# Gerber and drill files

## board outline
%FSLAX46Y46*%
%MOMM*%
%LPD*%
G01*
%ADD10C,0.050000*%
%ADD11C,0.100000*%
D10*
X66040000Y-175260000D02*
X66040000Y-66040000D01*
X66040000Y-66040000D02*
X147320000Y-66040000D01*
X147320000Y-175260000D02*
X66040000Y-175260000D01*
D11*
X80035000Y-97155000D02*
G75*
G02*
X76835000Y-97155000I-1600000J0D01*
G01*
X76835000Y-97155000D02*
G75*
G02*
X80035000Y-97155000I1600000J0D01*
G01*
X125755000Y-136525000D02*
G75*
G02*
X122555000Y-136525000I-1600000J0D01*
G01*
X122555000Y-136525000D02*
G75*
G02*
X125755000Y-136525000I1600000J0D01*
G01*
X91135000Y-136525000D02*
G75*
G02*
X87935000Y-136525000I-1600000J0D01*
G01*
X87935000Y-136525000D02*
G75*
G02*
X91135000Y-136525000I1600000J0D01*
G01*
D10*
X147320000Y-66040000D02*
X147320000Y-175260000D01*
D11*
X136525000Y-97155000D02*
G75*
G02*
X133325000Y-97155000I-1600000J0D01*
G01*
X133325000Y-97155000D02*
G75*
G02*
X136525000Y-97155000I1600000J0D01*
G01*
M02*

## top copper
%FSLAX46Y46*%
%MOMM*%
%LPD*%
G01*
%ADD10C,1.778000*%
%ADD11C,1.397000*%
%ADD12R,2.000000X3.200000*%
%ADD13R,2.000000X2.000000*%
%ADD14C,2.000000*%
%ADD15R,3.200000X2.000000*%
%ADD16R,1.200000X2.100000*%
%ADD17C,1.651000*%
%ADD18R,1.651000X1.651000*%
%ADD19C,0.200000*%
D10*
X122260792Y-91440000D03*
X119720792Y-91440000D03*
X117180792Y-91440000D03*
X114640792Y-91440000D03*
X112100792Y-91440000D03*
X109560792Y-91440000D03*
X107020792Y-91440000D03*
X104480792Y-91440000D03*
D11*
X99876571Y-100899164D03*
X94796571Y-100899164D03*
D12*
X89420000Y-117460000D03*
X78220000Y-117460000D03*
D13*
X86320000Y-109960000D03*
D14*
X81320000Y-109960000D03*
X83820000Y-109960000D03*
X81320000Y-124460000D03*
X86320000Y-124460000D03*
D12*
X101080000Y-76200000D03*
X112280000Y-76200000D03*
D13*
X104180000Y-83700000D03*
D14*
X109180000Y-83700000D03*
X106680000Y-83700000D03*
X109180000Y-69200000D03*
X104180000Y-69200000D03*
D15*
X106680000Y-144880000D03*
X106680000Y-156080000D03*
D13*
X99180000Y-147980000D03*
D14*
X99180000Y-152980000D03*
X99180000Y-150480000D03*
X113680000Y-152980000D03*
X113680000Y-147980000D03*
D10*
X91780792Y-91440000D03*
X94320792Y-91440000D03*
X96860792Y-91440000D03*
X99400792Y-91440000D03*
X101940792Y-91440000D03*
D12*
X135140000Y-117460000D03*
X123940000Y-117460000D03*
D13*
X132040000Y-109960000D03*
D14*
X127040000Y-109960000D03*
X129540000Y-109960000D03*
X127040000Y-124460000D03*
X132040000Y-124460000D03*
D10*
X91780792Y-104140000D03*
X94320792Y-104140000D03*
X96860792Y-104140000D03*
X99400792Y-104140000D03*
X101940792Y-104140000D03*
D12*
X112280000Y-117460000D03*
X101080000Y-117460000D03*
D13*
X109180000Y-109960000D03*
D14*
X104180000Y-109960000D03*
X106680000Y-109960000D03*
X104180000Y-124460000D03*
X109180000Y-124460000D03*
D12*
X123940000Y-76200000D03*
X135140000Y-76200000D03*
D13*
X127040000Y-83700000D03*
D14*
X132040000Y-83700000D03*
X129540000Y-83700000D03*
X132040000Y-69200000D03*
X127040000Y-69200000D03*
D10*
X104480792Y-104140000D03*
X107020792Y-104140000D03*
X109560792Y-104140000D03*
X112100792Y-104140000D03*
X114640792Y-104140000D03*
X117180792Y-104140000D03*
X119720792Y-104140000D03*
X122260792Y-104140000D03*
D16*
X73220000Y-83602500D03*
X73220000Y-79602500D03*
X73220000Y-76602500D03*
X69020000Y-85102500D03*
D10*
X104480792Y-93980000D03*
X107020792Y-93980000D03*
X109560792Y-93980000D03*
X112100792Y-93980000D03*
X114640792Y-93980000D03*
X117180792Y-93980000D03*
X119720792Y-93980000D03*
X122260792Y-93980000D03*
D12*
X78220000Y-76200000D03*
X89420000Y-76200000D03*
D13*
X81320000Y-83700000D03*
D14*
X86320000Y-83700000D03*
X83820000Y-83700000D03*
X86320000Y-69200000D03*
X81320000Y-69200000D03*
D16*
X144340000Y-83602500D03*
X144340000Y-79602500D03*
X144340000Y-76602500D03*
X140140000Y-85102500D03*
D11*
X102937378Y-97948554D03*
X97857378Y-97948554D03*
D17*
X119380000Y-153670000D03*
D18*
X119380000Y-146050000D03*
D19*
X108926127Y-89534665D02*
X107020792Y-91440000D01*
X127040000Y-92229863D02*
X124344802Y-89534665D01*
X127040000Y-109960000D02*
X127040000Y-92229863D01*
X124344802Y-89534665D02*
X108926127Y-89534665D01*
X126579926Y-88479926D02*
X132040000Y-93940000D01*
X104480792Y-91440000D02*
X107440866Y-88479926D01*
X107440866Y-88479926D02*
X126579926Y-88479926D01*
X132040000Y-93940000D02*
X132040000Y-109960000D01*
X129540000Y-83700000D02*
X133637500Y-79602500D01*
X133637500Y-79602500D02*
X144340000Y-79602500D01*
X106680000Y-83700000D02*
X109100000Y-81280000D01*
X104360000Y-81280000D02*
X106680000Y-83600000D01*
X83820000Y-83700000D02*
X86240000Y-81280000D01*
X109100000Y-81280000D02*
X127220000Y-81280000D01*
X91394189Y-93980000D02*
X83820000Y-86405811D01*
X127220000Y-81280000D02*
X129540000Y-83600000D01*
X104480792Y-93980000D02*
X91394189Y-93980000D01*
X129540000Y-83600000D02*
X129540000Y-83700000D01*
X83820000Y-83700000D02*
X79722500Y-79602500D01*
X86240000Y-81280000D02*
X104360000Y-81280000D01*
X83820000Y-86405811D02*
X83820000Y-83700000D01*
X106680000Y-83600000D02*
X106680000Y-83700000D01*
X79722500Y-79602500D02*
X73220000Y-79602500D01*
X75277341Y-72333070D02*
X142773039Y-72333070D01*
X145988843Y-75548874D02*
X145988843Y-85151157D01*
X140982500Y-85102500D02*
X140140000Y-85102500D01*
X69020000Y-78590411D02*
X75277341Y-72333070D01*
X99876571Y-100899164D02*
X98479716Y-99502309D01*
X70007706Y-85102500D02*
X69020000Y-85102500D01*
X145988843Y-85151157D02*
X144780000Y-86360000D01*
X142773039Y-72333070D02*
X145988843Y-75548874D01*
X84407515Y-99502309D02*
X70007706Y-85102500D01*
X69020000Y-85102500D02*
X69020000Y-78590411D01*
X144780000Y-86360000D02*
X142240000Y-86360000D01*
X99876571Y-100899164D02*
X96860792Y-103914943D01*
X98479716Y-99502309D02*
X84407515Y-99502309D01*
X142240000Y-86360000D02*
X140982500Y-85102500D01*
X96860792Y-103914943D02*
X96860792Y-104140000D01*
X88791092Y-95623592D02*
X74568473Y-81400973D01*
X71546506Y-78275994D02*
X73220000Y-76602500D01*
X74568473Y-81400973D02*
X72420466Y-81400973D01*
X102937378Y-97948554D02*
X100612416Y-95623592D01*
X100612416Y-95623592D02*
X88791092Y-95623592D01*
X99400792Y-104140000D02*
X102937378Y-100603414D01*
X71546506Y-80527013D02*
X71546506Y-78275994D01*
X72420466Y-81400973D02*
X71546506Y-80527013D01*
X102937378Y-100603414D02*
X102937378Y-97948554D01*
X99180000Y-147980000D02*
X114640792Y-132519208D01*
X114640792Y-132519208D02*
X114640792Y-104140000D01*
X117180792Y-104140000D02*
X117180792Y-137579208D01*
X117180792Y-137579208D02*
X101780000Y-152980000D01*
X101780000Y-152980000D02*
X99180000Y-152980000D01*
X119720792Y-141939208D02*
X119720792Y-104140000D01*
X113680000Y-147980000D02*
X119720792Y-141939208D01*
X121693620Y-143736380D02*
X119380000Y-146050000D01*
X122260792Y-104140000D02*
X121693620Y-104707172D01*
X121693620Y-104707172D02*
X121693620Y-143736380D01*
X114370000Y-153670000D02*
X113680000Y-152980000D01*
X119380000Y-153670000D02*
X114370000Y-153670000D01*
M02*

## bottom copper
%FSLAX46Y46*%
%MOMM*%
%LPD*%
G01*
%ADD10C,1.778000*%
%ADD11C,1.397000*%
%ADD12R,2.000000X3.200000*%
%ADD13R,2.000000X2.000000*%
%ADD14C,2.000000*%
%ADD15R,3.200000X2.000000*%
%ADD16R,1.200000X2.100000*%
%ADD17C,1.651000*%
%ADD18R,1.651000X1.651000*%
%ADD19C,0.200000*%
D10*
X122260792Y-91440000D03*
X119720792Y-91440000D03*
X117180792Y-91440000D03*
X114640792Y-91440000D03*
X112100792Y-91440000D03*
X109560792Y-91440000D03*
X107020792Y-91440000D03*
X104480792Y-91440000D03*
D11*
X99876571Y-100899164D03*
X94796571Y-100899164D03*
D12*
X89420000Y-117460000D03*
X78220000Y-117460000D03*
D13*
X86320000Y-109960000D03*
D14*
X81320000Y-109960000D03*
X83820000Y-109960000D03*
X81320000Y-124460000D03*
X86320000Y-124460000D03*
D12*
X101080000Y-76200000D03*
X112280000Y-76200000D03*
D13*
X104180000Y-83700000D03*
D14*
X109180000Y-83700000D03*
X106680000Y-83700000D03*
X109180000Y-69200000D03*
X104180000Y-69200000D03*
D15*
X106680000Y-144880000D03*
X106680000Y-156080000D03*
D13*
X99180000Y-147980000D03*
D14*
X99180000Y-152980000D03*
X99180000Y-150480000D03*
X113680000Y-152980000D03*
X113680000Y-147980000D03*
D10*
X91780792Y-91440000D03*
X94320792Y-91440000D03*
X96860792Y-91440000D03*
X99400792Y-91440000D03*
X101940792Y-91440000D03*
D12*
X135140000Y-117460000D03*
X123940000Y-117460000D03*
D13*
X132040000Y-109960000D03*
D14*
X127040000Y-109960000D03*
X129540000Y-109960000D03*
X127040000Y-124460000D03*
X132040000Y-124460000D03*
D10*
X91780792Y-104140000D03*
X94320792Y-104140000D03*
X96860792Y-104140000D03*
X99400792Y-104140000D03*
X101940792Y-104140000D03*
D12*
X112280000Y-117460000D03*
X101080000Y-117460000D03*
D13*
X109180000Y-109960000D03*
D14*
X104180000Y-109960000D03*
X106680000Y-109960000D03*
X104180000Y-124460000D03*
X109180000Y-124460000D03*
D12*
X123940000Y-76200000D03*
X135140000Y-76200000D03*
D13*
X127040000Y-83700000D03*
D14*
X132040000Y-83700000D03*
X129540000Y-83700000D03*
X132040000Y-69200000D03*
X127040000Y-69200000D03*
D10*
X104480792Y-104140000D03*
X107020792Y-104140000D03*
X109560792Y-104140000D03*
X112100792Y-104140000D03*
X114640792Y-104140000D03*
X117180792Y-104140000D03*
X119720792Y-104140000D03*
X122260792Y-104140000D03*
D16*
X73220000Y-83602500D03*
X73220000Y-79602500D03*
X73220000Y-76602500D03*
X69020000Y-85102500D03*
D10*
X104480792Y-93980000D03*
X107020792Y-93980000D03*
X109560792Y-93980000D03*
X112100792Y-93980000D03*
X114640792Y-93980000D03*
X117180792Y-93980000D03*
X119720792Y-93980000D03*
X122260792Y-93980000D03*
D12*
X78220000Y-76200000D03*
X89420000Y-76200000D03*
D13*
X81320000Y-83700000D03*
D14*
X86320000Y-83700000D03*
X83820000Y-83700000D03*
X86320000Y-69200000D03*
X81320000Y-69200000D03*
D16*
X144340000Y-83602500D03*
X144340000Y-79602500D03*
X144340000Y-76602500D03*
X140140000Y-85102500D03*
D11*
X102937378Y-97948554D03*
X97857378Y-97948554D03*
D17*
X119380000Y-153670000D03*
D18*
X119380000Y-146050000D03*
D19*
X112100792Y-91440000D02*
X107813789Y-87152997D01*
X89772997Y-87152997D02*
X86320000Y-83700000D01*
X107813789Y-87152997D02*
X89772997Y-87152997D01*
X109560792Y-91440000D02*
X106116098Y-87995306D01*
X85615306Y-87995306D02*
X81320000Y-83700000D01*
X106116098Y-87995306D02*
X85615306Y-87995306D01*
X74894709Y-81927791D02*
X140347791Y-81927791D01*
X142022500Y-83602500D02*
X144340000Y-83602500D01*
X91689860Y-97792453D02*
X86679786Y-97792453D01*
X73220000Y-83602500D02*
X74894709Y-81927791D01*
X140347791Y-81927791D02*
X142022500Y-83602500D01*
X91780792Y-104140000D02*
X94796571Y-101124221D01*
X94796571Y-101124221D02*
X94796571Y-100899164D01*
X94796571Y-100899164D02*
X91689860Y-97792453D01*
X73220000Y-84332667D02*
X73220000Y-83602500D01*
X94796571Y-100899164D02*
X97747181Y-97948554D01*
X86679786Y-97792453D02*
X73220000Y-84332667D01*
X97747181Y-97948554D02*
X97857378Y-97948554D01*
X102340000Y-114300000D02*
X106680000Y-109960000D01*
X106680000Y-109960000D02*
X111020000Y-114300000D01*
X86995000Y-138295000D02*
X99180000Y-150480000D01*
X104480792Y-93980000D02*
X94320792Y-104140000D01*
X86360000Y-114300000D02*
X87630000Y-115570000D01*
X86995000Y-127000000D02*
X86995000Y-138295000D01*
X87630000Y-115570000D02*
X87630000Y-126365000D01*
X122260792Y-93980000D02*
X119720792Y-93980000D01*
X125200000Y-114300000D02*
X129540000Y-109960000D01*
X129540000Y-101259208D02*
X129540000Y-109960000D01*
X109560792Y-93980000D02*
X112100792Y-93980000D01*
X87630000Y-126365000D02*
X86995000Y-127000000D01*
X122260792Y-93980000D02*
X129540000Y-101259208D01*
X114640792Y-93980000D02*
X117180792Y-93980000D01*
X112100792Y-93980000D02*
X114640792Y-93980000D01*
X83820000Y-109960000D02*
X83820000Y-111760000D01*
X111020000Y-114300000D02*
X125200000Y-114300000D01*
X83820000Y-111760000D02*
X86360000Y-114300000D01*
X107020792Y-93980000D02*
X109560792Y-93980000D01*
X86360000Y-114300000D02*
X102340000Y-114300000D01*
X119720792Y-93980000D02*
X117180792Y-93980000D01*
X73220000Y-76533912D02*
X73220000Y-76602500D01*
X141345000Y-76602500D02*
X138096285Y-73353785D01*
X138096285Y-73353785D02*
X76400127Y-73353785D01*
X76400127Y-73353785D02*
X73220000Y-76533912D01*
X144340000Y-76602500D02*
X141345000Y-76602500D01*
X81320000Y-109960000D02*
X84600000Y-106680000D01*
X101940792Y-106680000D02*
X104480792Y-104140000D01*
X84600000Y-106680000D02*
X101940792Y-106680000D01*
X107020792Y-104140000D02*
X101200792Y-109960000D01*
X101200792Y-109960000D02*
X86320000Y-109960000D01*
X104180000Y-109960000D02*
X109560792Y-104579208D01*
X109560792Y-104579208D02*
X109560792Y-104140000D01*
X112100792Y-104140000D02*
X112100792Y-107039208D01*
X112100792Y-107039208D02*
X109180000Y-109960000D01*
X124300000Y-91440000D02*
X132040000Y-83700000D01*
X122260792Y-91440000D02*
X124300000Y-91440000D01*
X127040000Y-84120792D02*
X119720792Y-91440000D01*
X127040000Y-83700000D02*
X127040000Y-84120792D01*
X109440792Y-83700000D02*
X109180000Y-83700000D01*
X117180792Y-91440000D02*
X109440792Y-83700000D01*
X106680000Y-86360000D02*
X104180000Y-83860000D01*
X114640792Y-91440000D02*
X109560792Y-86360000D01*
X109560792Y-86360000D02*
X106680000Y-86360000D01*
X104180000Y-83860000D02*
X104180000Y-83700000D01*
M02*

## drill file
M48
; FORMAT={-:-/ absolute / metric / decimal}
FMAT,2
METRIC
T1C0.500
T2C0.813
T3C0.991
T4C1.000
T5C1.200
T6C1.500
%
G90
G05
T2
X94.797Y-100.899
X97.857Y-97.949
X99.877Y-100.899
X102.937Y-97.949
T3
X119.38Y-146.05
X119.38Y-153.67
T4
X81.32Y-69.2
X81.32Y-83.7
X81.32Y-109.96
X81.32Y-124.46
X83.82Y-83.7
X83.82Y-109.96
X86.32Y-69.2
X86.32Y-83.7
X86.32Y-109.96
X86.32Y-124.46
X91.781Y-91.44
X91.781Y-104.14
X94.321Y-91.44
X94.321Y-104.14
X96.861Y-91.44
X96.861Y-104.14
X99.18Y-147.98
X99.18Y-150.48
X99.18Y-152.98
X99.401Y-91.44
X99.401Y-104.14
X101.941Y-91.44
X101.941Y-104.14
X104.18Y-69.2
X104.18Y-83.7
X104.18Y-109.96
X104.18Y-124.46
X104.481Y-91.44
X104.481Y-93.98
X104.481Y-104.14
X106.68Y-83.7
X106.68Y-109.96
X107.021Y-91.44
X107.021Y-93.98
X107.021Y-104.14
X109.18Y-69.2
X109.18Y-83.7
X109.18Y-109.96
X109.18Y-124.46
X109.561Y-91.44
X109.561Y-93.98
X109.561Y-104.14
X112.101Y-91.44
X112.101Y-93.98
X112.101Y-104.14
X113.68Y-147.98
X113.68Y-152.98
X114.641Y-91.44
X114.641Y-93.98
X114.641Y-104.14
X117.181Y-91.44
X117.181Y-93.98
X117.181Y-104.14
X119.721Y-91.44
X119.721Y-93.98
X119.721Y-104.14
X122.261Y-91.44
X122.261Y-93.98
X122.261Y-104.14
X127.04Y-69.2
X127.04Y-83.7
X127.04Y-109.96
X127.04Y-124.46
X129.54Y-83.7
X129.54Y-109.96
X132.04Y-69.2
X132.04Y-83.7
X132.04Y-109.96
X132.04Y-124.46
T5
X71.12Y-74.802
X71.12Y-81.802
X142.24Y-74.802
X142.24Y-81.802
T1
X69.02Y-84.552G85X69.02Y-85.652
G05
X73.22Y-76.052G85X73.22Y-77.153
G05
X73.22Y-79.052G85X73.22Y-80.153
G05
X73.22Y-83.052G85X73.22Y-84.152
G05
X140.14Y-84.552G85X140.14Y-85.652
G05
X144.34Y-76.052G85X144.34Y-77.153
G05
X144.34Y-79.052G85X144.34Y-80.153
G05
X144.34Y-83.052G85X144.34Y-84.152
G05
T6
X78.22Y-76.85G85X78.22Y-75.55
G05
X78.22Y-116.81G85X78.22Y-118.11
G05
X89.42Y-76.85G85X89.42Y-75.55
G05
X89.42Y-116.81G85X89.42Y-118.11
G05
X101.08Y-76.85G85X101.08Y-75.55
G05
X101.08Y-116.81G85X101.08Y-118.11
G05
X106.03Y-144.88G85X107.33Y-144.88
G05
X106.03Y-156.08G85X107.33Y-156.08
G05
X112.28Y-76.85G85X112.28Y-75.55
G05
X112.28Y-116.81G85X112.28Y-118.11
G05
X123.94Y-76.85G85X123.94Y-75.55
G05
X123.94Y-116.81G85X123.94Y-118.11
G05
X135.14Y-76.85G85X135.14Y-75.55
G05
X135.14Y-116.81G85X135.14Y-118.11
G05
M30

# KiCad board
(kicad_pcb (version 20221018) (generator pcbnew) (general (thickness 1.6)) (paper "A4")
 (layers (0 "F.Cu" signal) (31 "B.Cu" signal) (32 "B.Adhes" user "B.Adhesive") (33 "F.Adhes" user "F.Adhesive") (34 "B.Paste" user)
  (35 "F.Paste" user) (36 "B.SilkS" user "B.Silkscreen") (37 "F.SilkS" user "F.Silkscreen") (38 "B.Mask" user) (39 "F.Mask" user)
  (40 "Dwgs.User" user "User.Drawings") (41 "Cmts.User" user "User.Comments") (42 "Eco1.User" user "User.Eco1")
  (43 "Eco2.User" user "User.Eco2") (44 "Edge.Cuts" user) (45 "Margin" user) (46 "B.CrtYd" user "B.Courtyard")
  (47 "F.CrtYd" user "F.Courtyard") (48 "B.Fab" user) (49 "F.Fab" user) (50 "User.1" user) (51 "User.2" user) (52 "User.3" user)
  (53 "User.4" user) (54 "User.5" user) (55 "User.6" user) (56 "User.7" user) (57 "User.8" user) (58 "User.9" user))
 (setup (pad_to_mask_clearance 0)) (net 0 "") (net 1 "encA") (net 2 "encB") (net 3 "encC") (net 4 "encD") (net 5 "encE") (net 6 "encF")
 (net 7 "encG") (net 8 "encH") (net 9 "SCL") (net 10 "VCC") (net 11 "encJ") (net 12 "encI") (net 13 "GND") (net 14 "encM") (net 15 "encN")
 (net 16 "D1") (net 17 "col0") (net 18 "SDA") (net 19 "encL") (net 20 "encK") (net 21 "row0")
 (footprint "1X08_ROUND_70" (layer "F.Cu") (at 113.370792 91.44 180)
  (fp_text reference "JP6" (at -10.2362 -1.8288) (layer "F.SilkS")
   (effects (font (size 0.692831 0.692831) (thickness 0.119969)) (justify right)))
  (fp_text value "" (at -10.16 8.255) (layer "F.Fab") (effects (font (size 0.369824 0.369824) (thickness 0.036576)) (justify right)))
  (pad "1" thru_hole circle (at -8.89 0 270) (size 1.778 1.778) (drill 1) (layers "*.Cu" "*.Mask") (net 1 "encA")
   (solder_mask_margin 0.0508))
  (pad "2" thru_hole circle (at -6.35 0 270) (size 1.778 1.778) (drill 1) (layers "*.Cu" "*.Mask") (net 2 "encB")
   (solder_mask_margin 0.0508))
  (pad "3" thru_hole circle (at -3.81 0 270) (size 1.778 1.778) (drill 1) (layers "*.Cu" "*.Mask") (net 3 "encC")
   (solder_mask_margin 0.0508))
  (pad "4" thru_hole circle (at -1.27 0 270) (size 1.778 1.778) (drill 1) (layers "*.Cu" "*.Mask") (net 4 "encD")
   (solder_mask_margin 0.0508))
  (pad "5" thru_hole circle (at 1.27 0 270) (size 1.778 1.778) (drill 1) (layers "*.Cu" "*.Mask") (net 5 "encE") (solder_mask_margin 0.0508))
  (pad "6" thru_hole circle (at 3.81 0 270) (size 1.778 1.778) (drill 1) (layers "*.Cu" "*.Mask") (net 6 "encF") (solder_mask_margin 0.0508))
  (pad "7" thru_hole circle (at 6.35 0 270) (size 1.778 1.778) (drill 1) (layers "*.Cu" "*.Mask") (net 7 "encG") (solder_mask_margin 0.0508))
  (pad "8" thru_hole circle (at 8.89 0 270) (size 1.778 1.778) (drill 1) (layers "*.Cu" "*.Mask") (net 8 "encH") (solder_mask_margin 0.0508)))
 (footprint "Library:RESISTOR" (layer "F.Cu") (at 97.336571 100.899164 180)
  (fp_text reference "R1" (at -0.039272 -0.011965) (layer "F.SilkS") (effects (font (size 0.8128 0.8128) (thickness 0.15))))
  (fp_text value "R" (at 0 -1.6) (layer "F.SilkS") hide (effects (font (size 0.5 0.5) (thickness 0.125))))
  (pad "1" thru_hole circle (at -2.54 0 180) (size 1.397 1.397) (drill 0.8128) (layers "*.Cu" "*.Mask") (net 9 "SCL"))
  (pad "2" thru_hole circle (at 2.54 0 180) (size 1.397 1.397) (drill 0.8128) (layers "*.Cu" "*.Mask") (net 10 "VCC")))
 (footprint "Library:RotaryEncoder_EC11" (layer "F.Cu") (at 83.82 117.46 -90)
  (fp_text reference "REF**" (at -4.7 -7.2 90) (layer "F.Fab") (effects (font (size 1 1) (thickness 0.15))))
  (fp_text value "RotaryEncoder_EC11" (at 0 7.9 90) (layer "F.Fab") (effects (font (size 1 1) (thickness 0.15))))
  (pad "" np_thru_hole rect (at 0 -5.6 270) (size 3.2 2) (drill oval 2.8 1.5) (layers "*.Cu" "*.Mask"))
  (pad "" np_thru_hole rect (at 0 5.6 270) (size 3.2 2) (drill oval 2.8 1.5) (layers "*.Cu" "*.Mask"))
  (pad "A" thru_hole rect (at -7.5 -2.5 270) (size 2 2) (drill 1) (layers "*.Cu" "*.Mask") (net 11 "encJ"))
  (pad "B" thru_hole circle (at -7.5 2.5 270) (size 2 2) (drill 1) (layers "*.Cu" "*.Mask") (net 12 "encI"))
  (pad "C" thru_hole circle (at -7.5 0 270) (size 2 2) (drill 1) (layers "*.Cu" "*.Mask") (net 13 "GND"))
  (pad "S1" thru_hole circle (at 7 2.5 270) (size 2 2) (drill 1) (layers "*.Cu" "*.Mask"))
  (pad "S2" thru_hole circle (at 7 -2.5 270) (size 2 2) (drill 1) (layers "*.Cu" "*.Mask")))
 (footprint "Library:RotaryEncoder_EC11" (layer "F.Cu") (at 106.68 76.2 90)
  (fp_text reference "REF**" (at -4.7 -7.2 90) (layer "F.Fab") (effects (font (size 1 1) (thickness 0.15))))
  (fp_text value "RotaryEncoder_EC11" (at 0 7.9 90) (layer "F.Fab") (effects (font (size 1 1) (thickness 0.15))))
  (pad "" np_thru_hole rect (at 0 -5.6 90) (size 3.2 2) (drill oval 2.8 1.5) (layers "*.Cu" "*.Mask"))
  (pad "" np_thru_hole rect (at 0 5.6 90) (size 3.2 2) (drill oval 2.8 1.5) (layers "*.Cu" "*.Mask"))
  (pad "A" thru_hole rect (at -7.5 -2.5 90) (size 2 2) (drill 1) (layers "*.Cu" "*.Mask") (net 4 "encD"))
  (pad "B" thru_hole circle (at -7.5 2.5 90) (size 2 2) (drill 1) (layers "*.Cu" "*.Mask") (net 3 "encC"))
  (pad "C" thru_hole circle (at -7.5 0 90) (size 2 2) (drill 1) (layers "*.Cu" "*.Mask") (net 13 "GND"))
  (pad "S1" thru_hole circle (at 7 2.5 90) (size 2 2) (drill 1) (layers "*.Cu" "*.Mask"))
  (pad "S2" thru_hole circle (at 7 -2.5 90) (size 2 2) (drill 1) (layers "*.Cu" "*.Mask")))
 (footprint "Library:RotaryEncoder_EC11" (layer "F.Cu") (at 106.68 150.48)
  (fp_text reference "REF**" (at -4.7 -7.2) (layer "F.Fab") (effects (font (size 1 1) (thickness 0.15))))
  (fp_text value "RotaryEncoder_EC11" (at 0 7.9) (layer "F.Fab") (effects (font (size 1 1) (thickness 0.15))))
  (pad "" np_thru_hole rect (at 0 -5.6) (size 3.2 2) (drill oval 2.8 1.5) (layers "*.Cu" "*.Mask"))
  (pad "" np_thru_hole rect (at 0 5.6) (size 3.2 2) (drill oval 2.8 1.5) (layers "*.Cu" "*.Mask"))
  (pad "A" thru_hole rect (at -7.5 -2.5) (size 2 2) (drill 1) (layers "*.Cu" "*.Mask") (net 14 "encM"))
  (pad "B" thru_hole circle (at -7.5 2.5) (size 2 2) (drill 1) (layers "*.Cu" "*.Mask") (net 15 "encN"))
  (pad "C" thru_hole circle (at -7.5 0) (size 2 2) (drill 1) (layers "*.Cu" "*.Mask") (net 13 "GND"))
  (pad "S1" thru_hole circle (at 7 2.5) (size 2 2) (drill 1) (layers "*.Cu" "*.Mask") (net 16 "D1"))
  (pad "S2" thru_hole circle (at 7 -2.5) (size 2 2) (drill 1) (layers "*.Cu" "*.Mask") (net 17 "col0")))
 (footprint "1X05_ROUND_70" (layer "F.Cu") (at 96.860792 91.44)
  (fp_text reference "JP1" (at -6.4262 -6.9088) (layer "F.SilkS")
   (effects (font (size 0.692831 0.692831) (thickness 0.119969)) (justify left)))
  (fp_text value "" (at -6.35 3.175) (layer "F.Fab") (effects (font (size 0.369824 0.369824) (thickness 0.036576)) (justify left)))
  (pad "1" thru_hole circle (at -5.08 0 90) (size 1.778 1.778) (drill 1) (layers "*.Cu" "*.Mask") (solder_mask_margin 0.0508))
  (pad "2" thru_hole circle (at -2.54 0 90) (size 1.778 1.778) (drill 1) (layers "*.Cu" "*.Mask") (solder_mask_margin 0.0508))
  (pad "3" thru_hole circle (at 0 0 90) (size 1.778 1.778) (drill 1) (layers "*.Cu" "*.Mask") (solder_mask_margin 0.0508))
  (pad "4" thru_hole circle (at 2.54 0 90) (size 1.778 1.778) (drill 1) (layers "*.Cu" "*.Mask") (solder_mask_margin 0.0508))
  (pad "5" thru_hole circle (at 5.08 0 90) (size 1.778 1.778) (drill 1) (layers "*.Cu" "*.Mask") (solder_mask_margin 0.0508)))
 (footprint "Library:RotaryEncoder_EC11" (layer "F.Cu") (at 129.54 117.46 -90)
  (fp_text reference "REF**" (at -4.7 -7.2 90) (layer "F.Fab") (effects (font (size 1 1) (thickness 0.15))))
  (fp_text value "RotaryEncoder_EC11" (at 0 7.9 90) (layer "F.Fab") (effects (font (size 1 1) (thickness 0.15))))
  (pad "" np_thru_hole rect (at 0 -5.6 270) (size 3.2 2) (drill oval 2.8 1.5) (layers "*.Cu" "*.Mask"))
  (pad "" np_thru_hole rect (at 0 5.6 270) (size 3.2 2) (drill oval 2.8 1.5) (layers "*.Cu" "*.Mask"))
  (pad "A" thru_hole rect (at -7.5 -2.5 270) (size 2 2) (drill 1) (layers "*.Cu" "*.Mask") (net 8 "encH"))
  (pad "B" thru_hole circle (at -7.5 2.5 270) (size 2 2) (drill 1) (layers "*.Cu" "*.Mask") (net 7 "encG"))
  (pad "C" thru_hole circle (at -7.5 0 270) (size 2 2) (drill 1) (layers "*.Cu" "*.Mask") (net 13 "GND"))
  (pad "S1" thru_hole circle (at 7 2.5 270) (size 2 2) (drill 1) (layers "*.Cu" "*.Mask"))
  (pad "S2" thru_hole circle (at 7 -2.5 270) (size 2 2) (drill 1) (layers "*.Cu" "*.Mask")))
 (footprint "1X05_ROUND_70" (layer "F.Cu") (at 96.860792 104.14)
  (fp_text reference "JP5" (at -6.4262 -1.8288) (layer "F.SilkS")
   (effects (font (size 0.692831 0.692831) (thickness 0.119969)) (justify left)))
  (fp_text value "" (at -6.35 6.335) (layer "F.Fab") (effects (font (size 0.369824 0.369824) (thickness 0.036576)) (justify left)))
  (pad "1" thru_hole circle (at -5.08 0 90) (size 1.778 1.778) (drill 1) (layers "*.Cu" "*.Mask") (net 10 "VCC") (solder_mask_margin 0.0508))
  (pad "2" thru_hole circle (at -2.54 0 90) (size 1.778 1.778) (drill 1) (layers "*.Cu" "*.Mask") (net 13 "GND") (solder_mask_margin 0.0508))
  (pad "3" thru_hole circle (at 0 0 90) (size 1.778 1.778) (drill 1) (layers "*.Cu" "*.Mask") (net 9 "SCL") (solder_mask_margin 0.0508))
  (pad "4" thru_hole circle (at 2.54 0 90) (size 1.778 1.778) (drill 1) (layers "*.Cu" "*.Mask") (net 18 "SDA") (solder_mask_margin 0.0508))
  (pad "5" thru_hole circle (at 5.08 0 90) (size 1.778 1.778) (drill 1) (layers "*.Cu" "*.Mask") (solder_mask_margin 0.0508)))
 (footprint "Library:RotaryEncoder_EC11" (layer "F.Cu") (at 106.68 117.46 -90)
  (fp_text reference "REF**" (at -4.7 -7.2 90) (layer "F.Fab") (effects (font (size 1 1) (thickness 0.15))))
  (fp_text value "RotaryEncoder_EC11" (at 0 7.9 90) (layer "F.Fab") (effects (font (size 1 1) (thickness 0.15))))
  (pad "" np_thru_hole rect (at 0 -5.6 270) (size 3.2 2) (drill oval 2.8 1.5) (layers "*.Cu" "*.Mask"))
  (pad "" np_thru_hole rect (at 0 5.6 270) (size 3.2 2) (drill oval 2.8 1.5) (layers "*.Cu" "*.Mask"))
  (pad "A" thru_hole rect (at -7.5 -2.5 270) (size 2 2) (drill 1) (layers "*.Cu" "*.Mask") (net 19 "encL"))
  (pad "B" thru_hole circle (at -7.5 2.5 270) (size 2 2) (drill 1) (layers "*.Cu" "*.Mask") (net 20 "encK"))
  (pad "C" thru_hole circle (at -7.5 0 270) (size 2 2) (drill 1) (layers "*.Cu" "*.Mask") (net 13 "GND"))
  (pad "S1" thru_hole circle (at 7 2.5 270) (size 2 2) (drill 1) (layers "*.Cu" "*.Mask"))
  (pad "S2" thru_hole circle (at 7 -2.5 270) (size 2 2) (drill 1) (layers "*.Cu" "*.Mask")))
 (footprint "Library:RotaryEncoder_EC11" (layer "F.Cu") (at 129.54 76.2 90)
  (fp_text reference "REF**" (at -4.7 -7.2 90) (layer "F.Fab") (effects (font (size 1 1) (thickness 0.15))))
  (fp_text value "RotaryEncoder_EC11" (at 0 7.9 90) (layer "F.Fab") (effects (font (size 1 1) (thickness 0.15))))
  (pad "" np_thru_hole rect (at 0 -5.6 90) (size 3.2 2) (drill oval 2.8 1.5) (layers "*.Cu" "*.Mask"))
  (pad "" np_thru_hole rect (at 0 5.6 90) (size 3.2 2) (drill oval 2.8 1.5) (layers "*.Cu" "*.Mask"))
  (pad "A" thru_hole rect (at -7.5 -2.5 90) (size 2 2) (drill 1) (layers "*.Cu" "*.Mask") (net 2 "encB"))
  (pad "B" thru_hole circle (at -7.5 2.5 90) (size 2 2) (drill 1) (layers "*.Cu" "*.Mask") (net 1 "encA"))
  (pad "C" thru_hole circle (at -7.5 0 90) (size 2 2) (drill 1) (layers "*.Cu" "*.Mask") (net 13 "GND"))
  (pad "S1" thru_hole circle (at 7 2.5 90) (size 2 2) (drill 1) (layers "*.Cu" "*.Mask"))
  (pad "S2" thru_hole circle (at 7 -2.5 90) (size 2 2) (drill 1) (layers "*.Cu" "*.Mask")))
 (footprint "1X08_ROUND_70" (layer "F.Cu") (at 113.370792 104.14)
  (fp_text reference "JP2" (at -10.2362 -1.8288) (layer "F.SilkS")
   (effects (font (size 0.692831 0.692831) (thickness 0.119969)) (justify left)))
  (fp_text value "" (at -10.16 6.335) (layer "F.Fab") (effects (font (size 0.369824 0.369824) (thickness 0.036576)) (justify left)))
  (pad "1" thru_hole circle (at -8.89 0 90) (size 1.778 1.778) (drill 1) (layers "*.Cu" "*.Mask") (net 12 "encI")
   (solder_mask_margin 0.0508))
  (pad "2" thru_hole circle (at -6.35 0 90) (size 1.778 1.778) (drill 1) (layers "*.Cu" "*.Mask") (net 11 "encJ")
   (solder_mask_margin 0.0508))
  (pad "3" thru_hole circle (at -3.81 0 90) (size 1.778 1.778) (drill 1) (layers "*.Cu" "*.Mask") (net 20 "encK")
   (solder_mask_margin 0.0508))
  (pad "4" thru_hole circle (at -1.27 0 90) (size 1.778 1.778) (drill 1) (layers "*.Cu" "*.Mask") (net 19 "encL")
   (solder_mask_margin 0.0508))
  (pad "5" thru_hole circle (at 1.27 0 90) (size 1.778 1.778) (drill 1) (layers "*.Cu" "*.Mask") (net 14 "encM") (solder_mask_margin 0.0508))
  (pad "6" thru_hole circle (at 3.81 0 90) (size 1.778 1.778) (drill 1) (layers "*.Cu" "*.Mask") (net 15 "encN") (solder_mask_margin 0.0508))
  (pad "7" thru_hole circle (at 6.35 0 90) (size 1.778 1.778) (drill 1) (layers "*.Cu" "*.Mask") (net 17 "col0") (solder_mask_margin 0.0508))
  (pad "8" thru_hole circle (at 8.89 0 90) (size 1.778 1.778) (drill 1) (layers "*.Cu" "*.Mask") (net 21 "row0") (solder_mask_margin 0.0508)))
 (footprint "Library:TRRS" (layer "F.Cu") (at 71.12 73.3025)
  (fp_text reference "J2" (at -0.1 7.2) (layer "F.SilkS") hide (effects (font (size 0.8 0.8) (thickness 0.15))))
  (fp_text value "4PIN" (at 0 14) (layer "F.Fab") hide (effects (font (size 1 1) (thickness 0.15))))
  (pad "" np_thru_hole circle (at 0 1.5) (size 1.2 1.2) (drill 1.2) (layers "*.Cu" "*.Mask" "F.SilkS"))
  (pad "" np_thru_hole circle (at 0 8.5) (size 1.2 1.2) (drill 1.2) (layers "*.Cu" "*.Mask" "F.SilkS"))
  (pad "1" thru_hole rect (at 2.1 10.3) (size 1.2 2.1) (drill oval 0.5 1.6) (layers "*.Cu" "*.Mask" "F.SilkS") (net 10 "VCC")
   (clearance 0.15))
  (pad "2" thru_hole rect (at 2.1 6.3) (size 1.2 2.1) (drill oval 0.5 1.6) (layers "*.Cu" "*.Mask" "F.SilkS") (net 13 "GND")
   (clearance 0.15))
  (pad "3" thru_hole rect (at 2.1 3.3) (size 1.2 2.1) (drill oval 0.5 1.6) (layers "*.Cu" "*.Mask" "F.SilkS") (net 18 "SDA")
   (clearance 0.15))
  (pad "4" thru_hole rect (at -2.1 11.8) (size 1.2 2.1) (drill oval 0.5 1.6) (layers "*.Cu" "*.Mask" "F.SilkS") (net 9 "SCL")
   (clearance 0.15)))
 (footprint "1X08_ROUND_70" (layer "F.Cu") (at 113.370792 93.98)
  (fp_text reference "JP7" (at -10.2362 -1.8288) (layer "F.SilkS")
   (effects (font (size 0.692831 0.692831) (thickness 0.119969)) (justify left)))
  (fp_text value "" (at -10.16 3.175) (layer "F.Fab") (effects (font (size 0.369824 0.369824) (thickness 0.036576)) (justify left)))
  (pad "1" thru_hole circle (at -8.89 0 90) (size 1.778 1.778) (drill 1) (layers "*.Cu" "*.Mask") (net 13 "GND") (solder_mask_margin 0.0508))
  (pad "2" thru_hole circle (at -6.35 0 90) (size 1.778 1.778) (drill 1) (layers "*.Cu" "*.Mask") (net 13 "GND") (solder_mask_margin 0.0508))
  (pad "3" thru_hole circle (at -3.81 0 90) (size 1.778 1.778) (drill 1) (layers "*.Cu" "*.Mask") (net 13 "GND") (solder_mask_margin 0.0508))
  (pad "4" thru_hole circle (at -1.27 0 90) (size 1.778 1.778) (drill 1) (layers "*.Cu" "*.Mask") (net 13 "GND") (solder_mask_margin 0.0508))
  (pad "5" thru_hole circle (at 1.27 0 90) (size 1.778 1.778) (drill 1) (layers "*.Cu" "*.Mask") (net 13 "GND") (solder_mask_margin 0.0508))
  (pad "6" thru_hole circle (at 3.81 0 90) (size 1.778 1.778) (drill 1) (layers "*.Cu" "*.Mask") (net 13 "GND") (solder_mask_margin 0.0508))
  (pad "7" thru_hole circle (at 6.35 0 90) (size 1.778 1.778) (drill 1) (layers "*.Cu" "*.Mask") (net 13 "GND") (solder_mask_margin 0.0508))
  (pad "8" thru_hole circle (at 8.89 0 90) (size 1.778 1.778) (drill 1) (layers "*.Cu" "*.Mask") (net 13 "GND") (solder_mask_margin 0.0508)))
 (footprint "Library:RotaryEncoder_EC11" (layer "F.Cu") (at 83.82 76.2 90)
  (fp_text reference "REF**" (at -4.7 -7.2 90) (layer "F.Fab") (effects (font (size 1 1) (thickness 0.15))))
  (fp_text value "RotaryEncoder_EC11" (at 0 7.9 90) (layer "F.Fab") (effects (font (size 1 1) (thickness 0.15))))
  (pad "" np_thru_hole rect (at 0 -5.6 90) (size 3.2 2) (drill oval 2.8 1.5) (layers "*.Cu" "*.Mask"))
  (pad "" np_thru_hole rect (at 0 5.6 90) (size 3.2 2) (drill oval 2.8 1.5) (layers "*.Cu" "*.Mask"))
  (pad "A" thru_hole rect (at -7.5 -2.5 90) (size 2 2) (drill 1) (layers "*.Cu" "*.Mask") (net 6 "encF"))
  (pad "B" thru_hole circle (at -7.5 2.5 90) (size 2 2) (drill 1) (layers "*.Cu" "*.Mask") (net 5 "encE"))
  (pad "C" thru_hole circle (at -7.5 0 90) (size 2 2) (drill 1) (layers "*.Cu" "*.Mask") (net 13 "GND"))
  (pad "S1" thru_hole circle (at 7 2.5 90) (size 2 2) (drill 1) (layers "*.Cu" "*.Mask"))
  (pad "S2" thru_hole circle (at 7 -2.5 90) (size 2 2) (drill 1) (layers "*.Cu" "*.Mask")))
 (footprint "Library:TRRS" (layer "F.Cu") (at 142.24 73.3025)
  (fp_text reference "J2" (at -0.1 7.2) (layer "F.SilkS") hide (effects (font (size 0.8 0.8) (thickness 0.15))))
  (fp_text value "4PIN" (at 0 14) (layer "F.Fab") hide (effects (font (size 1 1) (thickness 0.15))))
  (pad "" np_thru_hole circle (at 0 1.5) (size 1.2 1.2) (drill 1.2) (layers "*.Cu" "*.Mask" "F.SilkS"))
  (pad "" np_thru_hole circle (at 0 8.5) (size 1.2 1.2) (drill 1.2) (layers "*.Cu" "*.Mask" "F.SilkS"))
  (pad "1" thru_hole rect (at 2.1 10.3) (size 1.2 2.1) (drill oval 0.5 1.6) (layers "*.Cu" "*.Mask" "F.SilkS") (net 10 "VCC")
   (clearance 0.15))
  (pad "2" thru_hole rect (at 2.1 6.3) (size 1.2 2.1) (drill oval 0.5 1.6) (layers "*.Cu" "*.Mask" "F.SilkS") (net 13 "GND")
   (clearance 0.15))
  (pad "3" thru_hole rect (at 2.1 3.3) (size 1.2 2.1) (drill oval 0.5 1.6) (layers "*.Cu" "*.Mask" "F.SilkS") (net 18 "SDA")
   (clearance 0.15))
  (pad "4" thru_hole rect (at -2.1 11.8) (size 1.2 2.1) (drill oval 0.5 1.6) (layers "*.Cu" "*.Mask" "F.SilkS") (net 9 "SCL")
   (clearance 0.15)))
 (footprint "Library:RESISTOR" (layer "F.Cu") (at 100.397378 97.948554 180)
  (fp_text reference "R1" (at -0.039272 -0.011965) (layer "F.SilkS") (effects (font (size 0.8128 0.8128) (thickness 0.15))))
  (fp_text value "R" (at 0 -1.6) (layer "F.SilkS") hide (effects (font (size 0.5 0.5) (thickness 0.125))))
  (pad "1" thru_hole circle (at -2.54 0 180) (size 1.397 1.397) (drill 0.8128) (layers "*.Cu" "*.Mask") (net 18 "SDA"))
  (pad "2" thru_hole circle (at 2.54 0 180) (size 1.397 1.397) (drill 0.8128) (layers "*.Cu" "*.Mask") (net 10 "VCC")))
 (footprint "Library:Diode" (layer "F.Cu") (at 119.38 149.86 90)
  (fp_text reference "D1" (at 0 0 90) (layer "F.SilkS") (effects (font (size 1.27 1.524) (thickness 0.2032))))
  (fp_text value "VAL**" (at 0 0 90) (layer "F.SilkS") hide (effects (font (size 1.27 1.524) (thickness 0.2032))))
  (pad "1" thru_hole circle (at -3.81 0 90) (size 1.651 1.651) (drill 0.9906) (layers "*.Cu" "*.SilkS" "*.Mask") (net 16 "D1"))
  (pad "2" thru_hole rect (at 3.81 0 90) (size 1.651 1.651) (drill 0.9906) (layers "*.Cu" "*.SilkS" "*.Mask") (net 21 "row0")))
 (gr_line (start 66.04 175.26) (end 66.04 66.04) (stroke (width 0.05) (type default)) (layer "Edge.Cuts"))
 (gr_line (start 66.04 66.04) (end 147.32 66.04) (stroke (width 0.05) (type default)) (layer "Edge.Cuts"))
 (gr_line (start 147.32 175.26) (end 66.04 175.26) (stroke (width 0.05) (type default)) (layer "Edge.Cuts"))
 (gr_circle (center 78.435 97.155) (end 80.035 97.155) (stroke (width 0.1) (type default)) (fill none) (layer "Edge.Cuts"))
 (gr_circle (center 124.155 136.525) (end 125.755 136.525) (stroke (width 0.1) (type default)) (fill none) (layer "Edge.Cuts"))
 (gr_circle (center 89.535 136.525) (end 91.135 136.525) (stroke (width 0.1) (type default)) (fill none) (layer "Edge.Cuts"))
 (gr_line (start 147.32 66.04) (end 147.32 175.26) (stroke (width 0.05) (type default)) (layer "Edge.Cuts"))
 (gr_circle (center 134.925 97.155) (end 136.525 97.155) (stroke (width 0.1) (type default)) (fill none) (layer "Edge.Cuts"))
 (segment (start 112.100792 91.44) (end 107.813789 87.152997) (width 0.2) (layer "B.Cu") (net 5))
 (segment (start 89.772997 87.152997) (end 86.32 83.7) (width 0.2) (layer "B.Cu") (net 5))
 (segment (start 107.813789 87.152997) (end 89.772997 87.152997) (width 0.2) (layer "B.Cu") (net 5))
 (segment (start 109.560792 91.44) (end 106.116098 87.995306) (width 0.2) (layer "B.Cu") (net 6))
 (segment (start 85.615306 87.995306) (end 81.32 83.7) (width 0.2) (layer "B.Cu") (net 6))
 (segment (start 106.116098 87.995306) (end 85.615306 87.995306) (width 0.2) (layer "B.Cu") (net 6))
 (segment (start 108.926127 89.534665) (end 107.020792 91.44) (width 0.2) (layer "F.Cu") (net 7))
 (segment (start 127.04 92.229863) (end 124.344802 89.534665) (width 0.2) (layer "F.Cu") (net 7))
 (segment (start 127.04 109.96) (end 127.04 92.229863) (width 0.2) (layer "F.Cu") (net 7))
 (segment (start 124.344802 89.534665) (end 108.926127 89.534665) (width 0.2) (layer "F.Cu") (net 7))
 (segment (start 126.579926 88.479926) (end 132.04 93.94) (width 0.2) (layer "F.Cu") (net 8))
 (segment (start 104.480792 91.44) (end 107.440866 88.479926) (width 0.2) (layer "F.Cu") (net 8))
 (segment (start 107.440866 88.479926) (end 126.579926 88.479926) (width 0.2) (layer "F.Cu") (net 8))
 (segment (start 132.04 93.94) (end 132.04 109.96) (width 0.2) (layer "F.Cu") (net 8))
 (segment (start 74.894709 81.927791) (end 140.347791 81.927791) (width 0.2) (layer "B.Cu") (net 10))
 (segment (start 142.0225 83.6025) (end 144.34 83.6025) (width 0.2) (layer "B.Cu") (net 10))
 (segment (start 91.68986 97.792453) (end 86.679786 97.792453) (width 0.2) (layer "B.Cu") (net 10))
 (segment (start 73.22 83.6025) (end 74.894709 81.927791) (width 0.2) (layer "B.Cu") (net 10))
 (segment (start 140.347791 81.927791) (end 142.0225 83.6025) (width 0.2) (layer "B.Cu") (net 10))
 (segment (start 91.780792 104.14) (end 94.796571 101.124221) (width 0.2) (layer "B.Cu") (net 10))
 (segment (start 94.796571 101.124221) (end 94.796571 100.899164) (width 0.2) (layer "B.Cu") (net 10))
 (segment (start 94.796571 100.899164) (end 91.68986 97.792453) (width 0.2) (layer "B.Cu") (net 10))
 (segment (start 73.22 84.332667) (end 73.22 83.6025) (width 0.2) (layer "B.Cu") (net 10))
 (segment (start 94.796571 100.899164) (end 97.747181 97.948554) (width 0.2) (layer "B.Cu") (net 10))
 (segment (start 86.679786 97.792453) (end 73.22 84.332667) (width 0.2) (layer "B.Cu") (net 10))
 (segment (start 97.747181 97.948554) (end 97.857378 97.948554) (width 0.2) (layer "B.Cu") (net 10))
 (segment (start 129.54 83.7) (end 133.6375 79.6025) (width 0.2) (layer "F.Cu") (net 13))
 (segment (start 133.6375 79.6025) (end 144.34 79.6025) (width 0.2) (layer "F.Cu") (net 13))
 (segment (start 106.68 83.7) (end 109.1 81.28) (width 0.2) (layer "F.Cu") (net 13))
 (segment (start 104.36 81.28) (end 106.68 83.6) (width 0.2) (layer "F.Cu") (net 13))
 (segment (start 83.82 83.7) (end 86.24 81.28) (width 0.2) (layer "F.Cu") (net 13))
 (segment (start 109.1 81.28) (end 127.22 81.28) (width 0.2) (layer "F.Cu") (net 13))
 (segment (start 91.394189 93.98) (end 83.82 86.405811) (width 0.2) (layer "F.Cu") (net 13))
 (segment (start 127.22 81.28) (end 129.54 83.6) (width 0.2) (layer "F.Cu") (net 13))
 (segment (start 104.480792 93.98) (end 91.394189 93.98) (width 0.2) (layer "F.Cu") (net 13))
 (segment (start 129.54 83.6) (end 129.54 83.7) (width 0.2) (layer "F.Cu") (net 13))
 (segment (start 83.82 83.7) (end 79.7225 79.6025) (width 0.2) (layer "F.Cu") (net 13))
 (segment (start 86.24 81.28) (end 104.36 81.28) (width 0.2) (layer "F.Cu") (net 13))
 (segment (start 83.82 86.405811) (end 83.82 83.7) (width 0.2) (layer "F.Cu") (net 13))
 (segment (start 106.68 83.6) (end 106.68 83.7) (width 0.2) (layer "F.Cu") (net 13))
 (segment (start 79.7225 79.6025) (end 73.22 79.6025) (width 0.2) (layer "F.Cu") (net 13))
 (segment (start 102.34 114.3) (end 106.68 109.96) (width 0.2) (layer "B.Cu") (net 13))
 (segment (start 106.68 109.96) (end 111.02 114.3) (width 0.2) (layer "B.Cu") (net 13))
 (segment (start 86.995 138.295) (end 99.18 150.48) (width 0.2) (layer "B.Cu") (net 13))
 (segment (start 104.480792 93.98) (end 94.320792 104.14) (width 0.2) (layer "B.Cu") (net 13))
 (segment (start 86.36 114.3) (end 87.63 115.57) (width 0.2) (layer "B.Cu") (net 13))
 (segment (start 86.995 127) (end 86.995 138.295) (width 0.2) (layer "B.Cu") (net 13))
 (segment (start 87.63 115.57) (end 87.63 126.365) (width 0.2) (layer "B.Cu") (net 13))
 (segment (start 122.260792 93.98) (end 119.720792 93.98) (width 0.2) (layer "B.Cu") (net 13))
 (segment (start 125.2 114.3) (end 129.54 109.96) (width 0.2) (layer "B.Cu") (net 13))
 (segment (start 129.54 101.259208) (end 129.54 109.96) (width 0.2) (layer "B.Cu") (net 13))
 (segment (start 109.560792 93.98) (end 112.100792 93.98) (width 0.2) (layer "B.Cu") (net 13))
 (segment (start 87.63 126.365) (end 86.995 127) (width 0.2) (layer "B.Cu") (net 13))
 (segment (start 122.260792 93.98) (end 129.54 101.259208) (width 0.2) (layer "B.Cu") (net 13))
 (segment (start 114.640792 93.98) (end 117.180792 93.98) (width 0.2) (layer "B.Cu") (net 13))
 (segment (start 112.100792 93.98) (end 114.640792 93.98) (width 0.2) (layer "B.Cu") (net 13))
 (segment (start 83.82 109.96) (end 83.82 111.76) (width 0.2) (layer "B.Cu") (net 13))
 (segment (start 111.02 114.3) (end 125.2 114.3) (width 0.2) (layer "B.Cu") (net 13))
 (segment (start 83.82 111.76) (end 86.36 114.3) (width 0.2) (layer "B.Cu") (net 13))
 (segment (start 107.020792 93.98) (end 109.560792 93.98) (width 0.2) (layer "B.Cu") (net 13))
 (segment (start 86.36 114.3) (end 102.34 114.3) (width 0.2) (layer "B.Cu") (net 13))
 (segment (start 119.720792 93.98) (end 117.180792 93.98) (width 0.2) (layer "B.Cu") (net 13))
 (segment (start 75.277341 72.33307) (end 142.773039 72.33307) (width 0.2) (layer "F.Cu") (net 9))
 (segment (start 145.988843 75.548874) (end 145.988843 85.151157) (width 0.2) (layer "F.Cu") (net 9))
 (segment (start 140.9825 85.1025) (end 140.14 85.1025) (width 0.2) (layer "F.Cu") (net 9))
 (segment (start 69.02 78.590411) (end 75.277341 72.33307) (width 0.2) (layer "F.Cu") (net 9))
 (segment (start 99.876571 100.899164) (end 98.479716 99.502309) (width 0.2) (layer "F.Cu") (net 9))
 (segment (start 70.007706 85.1025) (end 69.02 85.1025) (width 0.2) (layer "F.Cu") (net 9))
 (segment (start 145.988843 85.151157) (end 144.78 86.36) (width 0.2) (layer "F.Cu") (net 9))
 (segment (start 142.773039 72.33307) (end 145.988843 75.548874) (width 0.2) (layer "F.Cu") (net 9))
 (segment (start 84.407515 99.502309) (end 70.007706 85.1025) (width 0.2) (layer "F.Cu") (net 9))
 (segment (start 69.02 85.1025) (end 69.02 78.590411) (width 0.2) (layer "F.Cu") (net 9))
 (segment (start 144.78 86.36) (end 142.24 86.36) (width 0.2) (layer "F.Cu") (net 9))
 (segment (start 99.876571 100.899164) (end 96.860792 103.914943) (width 0.2) (layer "F.Cu") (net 9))
 (segment (start 98.479716 99.502309) (end 84.407515 99.502309) (width 0.2) (layer "F.Cu") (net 9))
 (segment (start 142.24 86.36) (end 140.9825 85.1025) (width 0.2) (layer "F.Cu") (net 9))
 (segment (start 96.860792 103.914943) (end 96.860792 104.14) (width 0.2) (layer "F.Cu") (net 9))
 (segment (start 88.791092 95.623592) (end 74.568473 81.400973) (width 0.2) (layer "F.Cu") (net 18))
 (segment (start 71.546506 78.275994) (end 73.22 76.6025) (width 0.2) (layer "F.Cu") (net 18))
 (segment (start 74.568473 81.400973) (end 72.420466 81.400973) (width 0.2) (layer "F.Cu") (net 18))
 (segment (start 102.937378 97.948554) (end 100.612416 95.623592) (width 0.2) (layer "F.Cu") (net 18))
 (segment (start 100.612416 95.623592) (end 88.791092 95.623592) (width 0.2) (layer "F.Cu") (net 18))
 (segment (start 99.400792 104.14) (end 102.937378 100.603414) (width 0.2) (layer "F.Cu") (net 18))
 (segment (start 71.546506 80.527013) (end 71.546506 78.275994) (width 0.2) (layer "F.Cu") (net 18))
 (segment (start 72.420466 81.400973) (end 71.546506 80.527013) (width 0.2) (layer "F.Cu") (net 18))
 (segment (start 102.937378 100.603414) (end 102.937378 97.948554) (width 0.2) (layer "F.Cu") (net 18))
 (segment (start 73.22 76.533912) (end 73.22 76.6025) (width 0.2) (layer "B.Cu") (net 18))
 (segment (start 141.345 76.6025) (end 138.096285 73.353785) (width 0.2) (layer "B.Cu") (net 18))
 (segment (start 138.096285 73.353785) (end 76.400127 73.353785) (width 0.2) (layer "B.Cu") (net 18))
 (segment (start 76.400127 73.353785) (end 73.22 76.533912) (width 0.2) (layer "B.Cu") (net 18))
 (segment (start 144.34 76.6025) (end 141.345 76.6025) (width 0.2) (layer "B.Cu") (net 18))
 (segment (start 81.32 109.96) (end 84.6 106.68) (width 0.2) (layer "B.Cu") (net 12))
 (segment (start 101.940792 106.68) (end 104.480792 104.14) (width 0.2) (layer "B.Cu") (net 12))
 (segment (start 84.6 106.68) (end 101.940792 106.68) (width 0.2) (layer "B.Cu") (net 12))
 (segment (start 107.020792 104.14) (end 101.200792 109.96) (width 0.2) (layer "B.Cu") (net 11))
 (segment (start 101.200792 109.96) (end 86.32 109.96) (width 0.2) (layer "B.Cu") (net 11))
 (segment (start 104.18 109.96) (end 109.560792 104.579208) (width 0.2) (layer "B.Cu") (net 20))
 (segment (start 109.560792 104.579208) (end 109.560792 104.14) (width 0.2) (layer "B.Cu") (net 20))
 (segment (start 112.100792 104.14) (end 112.100792 107.039208) (width 0.2) (layer "B.Cu") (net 19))
 (segment (start 112.100792 107.039208) (end 109.18 109.96) (width 0.2) (layer "B.Cu") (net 19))
 (segment (start 99.18 147.98) (end 114.640792 132.519208) (width 0.2) (layer "F.Cu") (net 14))
 (segment (start 114.640792 132.519208) (end 114.640792 104.14) (width 0.2) (layer "F.Cu") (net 14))
 (segment (start 117.180792 104.14) (end 117.180792 137.579208) (width 0.2) (layer "F.Cu") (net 15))
 (segment (start 117.180792 137.579208) (end 101.78 152.98) (width 0.2) (layer "F.Cu") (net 15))
 (segment (start 101.78 152.98) (end 99.18 152.98) (width 0.2) (layer "F.Cu") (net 15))
 (segment (start 119.720792 141.939208) (end 119.720792 104.14) (width 0.2) (layer "F.Cu") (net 17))
 (segment (start 113.68 147.98) (end 119.720792 141.939208) (width 0.2) (layer "F.Cu") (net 17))
 (segment (start 121.69362 143.73638) (end 119.38 146.05) (width 0.2) (layer "F.Cu") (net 21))
 (segment (start 122.260792 104.14) (end 121.69362 104.707172) (width 0.2) (layer "F.Cu") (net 21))
 (segment (start 121.69362 104.707172) (end 121.69362 143.73638) (width 0.2) (layer "F.Cu") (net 21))
 (segment (start 124.3 91.44) (end 132.04 83.7) (width 0.2) (layer "B.Cu") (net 1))
 (segment (start 122.260792 91.44) (end 124.3 91.44) (width 0.2) (layer "B.Cu") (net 1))
 (segment (start 127.04 84.120792) (end 119.720792 91.44) (width 0.2) (layer "B.Cu") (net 2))
 (segment (start 127.04 83.7) (end 127.04 84.120792) (width 0.2) (layer "B.Cu") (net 2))
 (segment (start 109.440792 83.7) (end 109.18 83.7) (width 0.2) (layer "B.Cu") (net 3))
 (segment (start 117.180792 91.44) (end 109.440792 83.7) (width 0.2) (layer "B.Cu") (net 3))
 (segment (start 106.68 86.36) (end 104.18 83.86) (width 0.2) (layer "B.Cu") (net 4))
 (segment (start 114.640792 91.44) (end 109.560792 86.36) (width 0.2) (layer "B.Cu") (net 4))
 (segment (start 109.560792 86.36) (end 106.68 86.36) (width 0.2) (layer "B.Cu") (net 4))
 (segment (start 104.18 83.86) (end 104.18 83.7) (width 0.2) (layer "B.Cu") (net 4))
 (segment (start 114.37 153.67) (end 113.68 152.98) (width 0.2) (layer "F.Cu") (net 16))
 (segment (start 119.38 153.67) (end 114.37 153.67) (width 0.2) (layer "F.Cu") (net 16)))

